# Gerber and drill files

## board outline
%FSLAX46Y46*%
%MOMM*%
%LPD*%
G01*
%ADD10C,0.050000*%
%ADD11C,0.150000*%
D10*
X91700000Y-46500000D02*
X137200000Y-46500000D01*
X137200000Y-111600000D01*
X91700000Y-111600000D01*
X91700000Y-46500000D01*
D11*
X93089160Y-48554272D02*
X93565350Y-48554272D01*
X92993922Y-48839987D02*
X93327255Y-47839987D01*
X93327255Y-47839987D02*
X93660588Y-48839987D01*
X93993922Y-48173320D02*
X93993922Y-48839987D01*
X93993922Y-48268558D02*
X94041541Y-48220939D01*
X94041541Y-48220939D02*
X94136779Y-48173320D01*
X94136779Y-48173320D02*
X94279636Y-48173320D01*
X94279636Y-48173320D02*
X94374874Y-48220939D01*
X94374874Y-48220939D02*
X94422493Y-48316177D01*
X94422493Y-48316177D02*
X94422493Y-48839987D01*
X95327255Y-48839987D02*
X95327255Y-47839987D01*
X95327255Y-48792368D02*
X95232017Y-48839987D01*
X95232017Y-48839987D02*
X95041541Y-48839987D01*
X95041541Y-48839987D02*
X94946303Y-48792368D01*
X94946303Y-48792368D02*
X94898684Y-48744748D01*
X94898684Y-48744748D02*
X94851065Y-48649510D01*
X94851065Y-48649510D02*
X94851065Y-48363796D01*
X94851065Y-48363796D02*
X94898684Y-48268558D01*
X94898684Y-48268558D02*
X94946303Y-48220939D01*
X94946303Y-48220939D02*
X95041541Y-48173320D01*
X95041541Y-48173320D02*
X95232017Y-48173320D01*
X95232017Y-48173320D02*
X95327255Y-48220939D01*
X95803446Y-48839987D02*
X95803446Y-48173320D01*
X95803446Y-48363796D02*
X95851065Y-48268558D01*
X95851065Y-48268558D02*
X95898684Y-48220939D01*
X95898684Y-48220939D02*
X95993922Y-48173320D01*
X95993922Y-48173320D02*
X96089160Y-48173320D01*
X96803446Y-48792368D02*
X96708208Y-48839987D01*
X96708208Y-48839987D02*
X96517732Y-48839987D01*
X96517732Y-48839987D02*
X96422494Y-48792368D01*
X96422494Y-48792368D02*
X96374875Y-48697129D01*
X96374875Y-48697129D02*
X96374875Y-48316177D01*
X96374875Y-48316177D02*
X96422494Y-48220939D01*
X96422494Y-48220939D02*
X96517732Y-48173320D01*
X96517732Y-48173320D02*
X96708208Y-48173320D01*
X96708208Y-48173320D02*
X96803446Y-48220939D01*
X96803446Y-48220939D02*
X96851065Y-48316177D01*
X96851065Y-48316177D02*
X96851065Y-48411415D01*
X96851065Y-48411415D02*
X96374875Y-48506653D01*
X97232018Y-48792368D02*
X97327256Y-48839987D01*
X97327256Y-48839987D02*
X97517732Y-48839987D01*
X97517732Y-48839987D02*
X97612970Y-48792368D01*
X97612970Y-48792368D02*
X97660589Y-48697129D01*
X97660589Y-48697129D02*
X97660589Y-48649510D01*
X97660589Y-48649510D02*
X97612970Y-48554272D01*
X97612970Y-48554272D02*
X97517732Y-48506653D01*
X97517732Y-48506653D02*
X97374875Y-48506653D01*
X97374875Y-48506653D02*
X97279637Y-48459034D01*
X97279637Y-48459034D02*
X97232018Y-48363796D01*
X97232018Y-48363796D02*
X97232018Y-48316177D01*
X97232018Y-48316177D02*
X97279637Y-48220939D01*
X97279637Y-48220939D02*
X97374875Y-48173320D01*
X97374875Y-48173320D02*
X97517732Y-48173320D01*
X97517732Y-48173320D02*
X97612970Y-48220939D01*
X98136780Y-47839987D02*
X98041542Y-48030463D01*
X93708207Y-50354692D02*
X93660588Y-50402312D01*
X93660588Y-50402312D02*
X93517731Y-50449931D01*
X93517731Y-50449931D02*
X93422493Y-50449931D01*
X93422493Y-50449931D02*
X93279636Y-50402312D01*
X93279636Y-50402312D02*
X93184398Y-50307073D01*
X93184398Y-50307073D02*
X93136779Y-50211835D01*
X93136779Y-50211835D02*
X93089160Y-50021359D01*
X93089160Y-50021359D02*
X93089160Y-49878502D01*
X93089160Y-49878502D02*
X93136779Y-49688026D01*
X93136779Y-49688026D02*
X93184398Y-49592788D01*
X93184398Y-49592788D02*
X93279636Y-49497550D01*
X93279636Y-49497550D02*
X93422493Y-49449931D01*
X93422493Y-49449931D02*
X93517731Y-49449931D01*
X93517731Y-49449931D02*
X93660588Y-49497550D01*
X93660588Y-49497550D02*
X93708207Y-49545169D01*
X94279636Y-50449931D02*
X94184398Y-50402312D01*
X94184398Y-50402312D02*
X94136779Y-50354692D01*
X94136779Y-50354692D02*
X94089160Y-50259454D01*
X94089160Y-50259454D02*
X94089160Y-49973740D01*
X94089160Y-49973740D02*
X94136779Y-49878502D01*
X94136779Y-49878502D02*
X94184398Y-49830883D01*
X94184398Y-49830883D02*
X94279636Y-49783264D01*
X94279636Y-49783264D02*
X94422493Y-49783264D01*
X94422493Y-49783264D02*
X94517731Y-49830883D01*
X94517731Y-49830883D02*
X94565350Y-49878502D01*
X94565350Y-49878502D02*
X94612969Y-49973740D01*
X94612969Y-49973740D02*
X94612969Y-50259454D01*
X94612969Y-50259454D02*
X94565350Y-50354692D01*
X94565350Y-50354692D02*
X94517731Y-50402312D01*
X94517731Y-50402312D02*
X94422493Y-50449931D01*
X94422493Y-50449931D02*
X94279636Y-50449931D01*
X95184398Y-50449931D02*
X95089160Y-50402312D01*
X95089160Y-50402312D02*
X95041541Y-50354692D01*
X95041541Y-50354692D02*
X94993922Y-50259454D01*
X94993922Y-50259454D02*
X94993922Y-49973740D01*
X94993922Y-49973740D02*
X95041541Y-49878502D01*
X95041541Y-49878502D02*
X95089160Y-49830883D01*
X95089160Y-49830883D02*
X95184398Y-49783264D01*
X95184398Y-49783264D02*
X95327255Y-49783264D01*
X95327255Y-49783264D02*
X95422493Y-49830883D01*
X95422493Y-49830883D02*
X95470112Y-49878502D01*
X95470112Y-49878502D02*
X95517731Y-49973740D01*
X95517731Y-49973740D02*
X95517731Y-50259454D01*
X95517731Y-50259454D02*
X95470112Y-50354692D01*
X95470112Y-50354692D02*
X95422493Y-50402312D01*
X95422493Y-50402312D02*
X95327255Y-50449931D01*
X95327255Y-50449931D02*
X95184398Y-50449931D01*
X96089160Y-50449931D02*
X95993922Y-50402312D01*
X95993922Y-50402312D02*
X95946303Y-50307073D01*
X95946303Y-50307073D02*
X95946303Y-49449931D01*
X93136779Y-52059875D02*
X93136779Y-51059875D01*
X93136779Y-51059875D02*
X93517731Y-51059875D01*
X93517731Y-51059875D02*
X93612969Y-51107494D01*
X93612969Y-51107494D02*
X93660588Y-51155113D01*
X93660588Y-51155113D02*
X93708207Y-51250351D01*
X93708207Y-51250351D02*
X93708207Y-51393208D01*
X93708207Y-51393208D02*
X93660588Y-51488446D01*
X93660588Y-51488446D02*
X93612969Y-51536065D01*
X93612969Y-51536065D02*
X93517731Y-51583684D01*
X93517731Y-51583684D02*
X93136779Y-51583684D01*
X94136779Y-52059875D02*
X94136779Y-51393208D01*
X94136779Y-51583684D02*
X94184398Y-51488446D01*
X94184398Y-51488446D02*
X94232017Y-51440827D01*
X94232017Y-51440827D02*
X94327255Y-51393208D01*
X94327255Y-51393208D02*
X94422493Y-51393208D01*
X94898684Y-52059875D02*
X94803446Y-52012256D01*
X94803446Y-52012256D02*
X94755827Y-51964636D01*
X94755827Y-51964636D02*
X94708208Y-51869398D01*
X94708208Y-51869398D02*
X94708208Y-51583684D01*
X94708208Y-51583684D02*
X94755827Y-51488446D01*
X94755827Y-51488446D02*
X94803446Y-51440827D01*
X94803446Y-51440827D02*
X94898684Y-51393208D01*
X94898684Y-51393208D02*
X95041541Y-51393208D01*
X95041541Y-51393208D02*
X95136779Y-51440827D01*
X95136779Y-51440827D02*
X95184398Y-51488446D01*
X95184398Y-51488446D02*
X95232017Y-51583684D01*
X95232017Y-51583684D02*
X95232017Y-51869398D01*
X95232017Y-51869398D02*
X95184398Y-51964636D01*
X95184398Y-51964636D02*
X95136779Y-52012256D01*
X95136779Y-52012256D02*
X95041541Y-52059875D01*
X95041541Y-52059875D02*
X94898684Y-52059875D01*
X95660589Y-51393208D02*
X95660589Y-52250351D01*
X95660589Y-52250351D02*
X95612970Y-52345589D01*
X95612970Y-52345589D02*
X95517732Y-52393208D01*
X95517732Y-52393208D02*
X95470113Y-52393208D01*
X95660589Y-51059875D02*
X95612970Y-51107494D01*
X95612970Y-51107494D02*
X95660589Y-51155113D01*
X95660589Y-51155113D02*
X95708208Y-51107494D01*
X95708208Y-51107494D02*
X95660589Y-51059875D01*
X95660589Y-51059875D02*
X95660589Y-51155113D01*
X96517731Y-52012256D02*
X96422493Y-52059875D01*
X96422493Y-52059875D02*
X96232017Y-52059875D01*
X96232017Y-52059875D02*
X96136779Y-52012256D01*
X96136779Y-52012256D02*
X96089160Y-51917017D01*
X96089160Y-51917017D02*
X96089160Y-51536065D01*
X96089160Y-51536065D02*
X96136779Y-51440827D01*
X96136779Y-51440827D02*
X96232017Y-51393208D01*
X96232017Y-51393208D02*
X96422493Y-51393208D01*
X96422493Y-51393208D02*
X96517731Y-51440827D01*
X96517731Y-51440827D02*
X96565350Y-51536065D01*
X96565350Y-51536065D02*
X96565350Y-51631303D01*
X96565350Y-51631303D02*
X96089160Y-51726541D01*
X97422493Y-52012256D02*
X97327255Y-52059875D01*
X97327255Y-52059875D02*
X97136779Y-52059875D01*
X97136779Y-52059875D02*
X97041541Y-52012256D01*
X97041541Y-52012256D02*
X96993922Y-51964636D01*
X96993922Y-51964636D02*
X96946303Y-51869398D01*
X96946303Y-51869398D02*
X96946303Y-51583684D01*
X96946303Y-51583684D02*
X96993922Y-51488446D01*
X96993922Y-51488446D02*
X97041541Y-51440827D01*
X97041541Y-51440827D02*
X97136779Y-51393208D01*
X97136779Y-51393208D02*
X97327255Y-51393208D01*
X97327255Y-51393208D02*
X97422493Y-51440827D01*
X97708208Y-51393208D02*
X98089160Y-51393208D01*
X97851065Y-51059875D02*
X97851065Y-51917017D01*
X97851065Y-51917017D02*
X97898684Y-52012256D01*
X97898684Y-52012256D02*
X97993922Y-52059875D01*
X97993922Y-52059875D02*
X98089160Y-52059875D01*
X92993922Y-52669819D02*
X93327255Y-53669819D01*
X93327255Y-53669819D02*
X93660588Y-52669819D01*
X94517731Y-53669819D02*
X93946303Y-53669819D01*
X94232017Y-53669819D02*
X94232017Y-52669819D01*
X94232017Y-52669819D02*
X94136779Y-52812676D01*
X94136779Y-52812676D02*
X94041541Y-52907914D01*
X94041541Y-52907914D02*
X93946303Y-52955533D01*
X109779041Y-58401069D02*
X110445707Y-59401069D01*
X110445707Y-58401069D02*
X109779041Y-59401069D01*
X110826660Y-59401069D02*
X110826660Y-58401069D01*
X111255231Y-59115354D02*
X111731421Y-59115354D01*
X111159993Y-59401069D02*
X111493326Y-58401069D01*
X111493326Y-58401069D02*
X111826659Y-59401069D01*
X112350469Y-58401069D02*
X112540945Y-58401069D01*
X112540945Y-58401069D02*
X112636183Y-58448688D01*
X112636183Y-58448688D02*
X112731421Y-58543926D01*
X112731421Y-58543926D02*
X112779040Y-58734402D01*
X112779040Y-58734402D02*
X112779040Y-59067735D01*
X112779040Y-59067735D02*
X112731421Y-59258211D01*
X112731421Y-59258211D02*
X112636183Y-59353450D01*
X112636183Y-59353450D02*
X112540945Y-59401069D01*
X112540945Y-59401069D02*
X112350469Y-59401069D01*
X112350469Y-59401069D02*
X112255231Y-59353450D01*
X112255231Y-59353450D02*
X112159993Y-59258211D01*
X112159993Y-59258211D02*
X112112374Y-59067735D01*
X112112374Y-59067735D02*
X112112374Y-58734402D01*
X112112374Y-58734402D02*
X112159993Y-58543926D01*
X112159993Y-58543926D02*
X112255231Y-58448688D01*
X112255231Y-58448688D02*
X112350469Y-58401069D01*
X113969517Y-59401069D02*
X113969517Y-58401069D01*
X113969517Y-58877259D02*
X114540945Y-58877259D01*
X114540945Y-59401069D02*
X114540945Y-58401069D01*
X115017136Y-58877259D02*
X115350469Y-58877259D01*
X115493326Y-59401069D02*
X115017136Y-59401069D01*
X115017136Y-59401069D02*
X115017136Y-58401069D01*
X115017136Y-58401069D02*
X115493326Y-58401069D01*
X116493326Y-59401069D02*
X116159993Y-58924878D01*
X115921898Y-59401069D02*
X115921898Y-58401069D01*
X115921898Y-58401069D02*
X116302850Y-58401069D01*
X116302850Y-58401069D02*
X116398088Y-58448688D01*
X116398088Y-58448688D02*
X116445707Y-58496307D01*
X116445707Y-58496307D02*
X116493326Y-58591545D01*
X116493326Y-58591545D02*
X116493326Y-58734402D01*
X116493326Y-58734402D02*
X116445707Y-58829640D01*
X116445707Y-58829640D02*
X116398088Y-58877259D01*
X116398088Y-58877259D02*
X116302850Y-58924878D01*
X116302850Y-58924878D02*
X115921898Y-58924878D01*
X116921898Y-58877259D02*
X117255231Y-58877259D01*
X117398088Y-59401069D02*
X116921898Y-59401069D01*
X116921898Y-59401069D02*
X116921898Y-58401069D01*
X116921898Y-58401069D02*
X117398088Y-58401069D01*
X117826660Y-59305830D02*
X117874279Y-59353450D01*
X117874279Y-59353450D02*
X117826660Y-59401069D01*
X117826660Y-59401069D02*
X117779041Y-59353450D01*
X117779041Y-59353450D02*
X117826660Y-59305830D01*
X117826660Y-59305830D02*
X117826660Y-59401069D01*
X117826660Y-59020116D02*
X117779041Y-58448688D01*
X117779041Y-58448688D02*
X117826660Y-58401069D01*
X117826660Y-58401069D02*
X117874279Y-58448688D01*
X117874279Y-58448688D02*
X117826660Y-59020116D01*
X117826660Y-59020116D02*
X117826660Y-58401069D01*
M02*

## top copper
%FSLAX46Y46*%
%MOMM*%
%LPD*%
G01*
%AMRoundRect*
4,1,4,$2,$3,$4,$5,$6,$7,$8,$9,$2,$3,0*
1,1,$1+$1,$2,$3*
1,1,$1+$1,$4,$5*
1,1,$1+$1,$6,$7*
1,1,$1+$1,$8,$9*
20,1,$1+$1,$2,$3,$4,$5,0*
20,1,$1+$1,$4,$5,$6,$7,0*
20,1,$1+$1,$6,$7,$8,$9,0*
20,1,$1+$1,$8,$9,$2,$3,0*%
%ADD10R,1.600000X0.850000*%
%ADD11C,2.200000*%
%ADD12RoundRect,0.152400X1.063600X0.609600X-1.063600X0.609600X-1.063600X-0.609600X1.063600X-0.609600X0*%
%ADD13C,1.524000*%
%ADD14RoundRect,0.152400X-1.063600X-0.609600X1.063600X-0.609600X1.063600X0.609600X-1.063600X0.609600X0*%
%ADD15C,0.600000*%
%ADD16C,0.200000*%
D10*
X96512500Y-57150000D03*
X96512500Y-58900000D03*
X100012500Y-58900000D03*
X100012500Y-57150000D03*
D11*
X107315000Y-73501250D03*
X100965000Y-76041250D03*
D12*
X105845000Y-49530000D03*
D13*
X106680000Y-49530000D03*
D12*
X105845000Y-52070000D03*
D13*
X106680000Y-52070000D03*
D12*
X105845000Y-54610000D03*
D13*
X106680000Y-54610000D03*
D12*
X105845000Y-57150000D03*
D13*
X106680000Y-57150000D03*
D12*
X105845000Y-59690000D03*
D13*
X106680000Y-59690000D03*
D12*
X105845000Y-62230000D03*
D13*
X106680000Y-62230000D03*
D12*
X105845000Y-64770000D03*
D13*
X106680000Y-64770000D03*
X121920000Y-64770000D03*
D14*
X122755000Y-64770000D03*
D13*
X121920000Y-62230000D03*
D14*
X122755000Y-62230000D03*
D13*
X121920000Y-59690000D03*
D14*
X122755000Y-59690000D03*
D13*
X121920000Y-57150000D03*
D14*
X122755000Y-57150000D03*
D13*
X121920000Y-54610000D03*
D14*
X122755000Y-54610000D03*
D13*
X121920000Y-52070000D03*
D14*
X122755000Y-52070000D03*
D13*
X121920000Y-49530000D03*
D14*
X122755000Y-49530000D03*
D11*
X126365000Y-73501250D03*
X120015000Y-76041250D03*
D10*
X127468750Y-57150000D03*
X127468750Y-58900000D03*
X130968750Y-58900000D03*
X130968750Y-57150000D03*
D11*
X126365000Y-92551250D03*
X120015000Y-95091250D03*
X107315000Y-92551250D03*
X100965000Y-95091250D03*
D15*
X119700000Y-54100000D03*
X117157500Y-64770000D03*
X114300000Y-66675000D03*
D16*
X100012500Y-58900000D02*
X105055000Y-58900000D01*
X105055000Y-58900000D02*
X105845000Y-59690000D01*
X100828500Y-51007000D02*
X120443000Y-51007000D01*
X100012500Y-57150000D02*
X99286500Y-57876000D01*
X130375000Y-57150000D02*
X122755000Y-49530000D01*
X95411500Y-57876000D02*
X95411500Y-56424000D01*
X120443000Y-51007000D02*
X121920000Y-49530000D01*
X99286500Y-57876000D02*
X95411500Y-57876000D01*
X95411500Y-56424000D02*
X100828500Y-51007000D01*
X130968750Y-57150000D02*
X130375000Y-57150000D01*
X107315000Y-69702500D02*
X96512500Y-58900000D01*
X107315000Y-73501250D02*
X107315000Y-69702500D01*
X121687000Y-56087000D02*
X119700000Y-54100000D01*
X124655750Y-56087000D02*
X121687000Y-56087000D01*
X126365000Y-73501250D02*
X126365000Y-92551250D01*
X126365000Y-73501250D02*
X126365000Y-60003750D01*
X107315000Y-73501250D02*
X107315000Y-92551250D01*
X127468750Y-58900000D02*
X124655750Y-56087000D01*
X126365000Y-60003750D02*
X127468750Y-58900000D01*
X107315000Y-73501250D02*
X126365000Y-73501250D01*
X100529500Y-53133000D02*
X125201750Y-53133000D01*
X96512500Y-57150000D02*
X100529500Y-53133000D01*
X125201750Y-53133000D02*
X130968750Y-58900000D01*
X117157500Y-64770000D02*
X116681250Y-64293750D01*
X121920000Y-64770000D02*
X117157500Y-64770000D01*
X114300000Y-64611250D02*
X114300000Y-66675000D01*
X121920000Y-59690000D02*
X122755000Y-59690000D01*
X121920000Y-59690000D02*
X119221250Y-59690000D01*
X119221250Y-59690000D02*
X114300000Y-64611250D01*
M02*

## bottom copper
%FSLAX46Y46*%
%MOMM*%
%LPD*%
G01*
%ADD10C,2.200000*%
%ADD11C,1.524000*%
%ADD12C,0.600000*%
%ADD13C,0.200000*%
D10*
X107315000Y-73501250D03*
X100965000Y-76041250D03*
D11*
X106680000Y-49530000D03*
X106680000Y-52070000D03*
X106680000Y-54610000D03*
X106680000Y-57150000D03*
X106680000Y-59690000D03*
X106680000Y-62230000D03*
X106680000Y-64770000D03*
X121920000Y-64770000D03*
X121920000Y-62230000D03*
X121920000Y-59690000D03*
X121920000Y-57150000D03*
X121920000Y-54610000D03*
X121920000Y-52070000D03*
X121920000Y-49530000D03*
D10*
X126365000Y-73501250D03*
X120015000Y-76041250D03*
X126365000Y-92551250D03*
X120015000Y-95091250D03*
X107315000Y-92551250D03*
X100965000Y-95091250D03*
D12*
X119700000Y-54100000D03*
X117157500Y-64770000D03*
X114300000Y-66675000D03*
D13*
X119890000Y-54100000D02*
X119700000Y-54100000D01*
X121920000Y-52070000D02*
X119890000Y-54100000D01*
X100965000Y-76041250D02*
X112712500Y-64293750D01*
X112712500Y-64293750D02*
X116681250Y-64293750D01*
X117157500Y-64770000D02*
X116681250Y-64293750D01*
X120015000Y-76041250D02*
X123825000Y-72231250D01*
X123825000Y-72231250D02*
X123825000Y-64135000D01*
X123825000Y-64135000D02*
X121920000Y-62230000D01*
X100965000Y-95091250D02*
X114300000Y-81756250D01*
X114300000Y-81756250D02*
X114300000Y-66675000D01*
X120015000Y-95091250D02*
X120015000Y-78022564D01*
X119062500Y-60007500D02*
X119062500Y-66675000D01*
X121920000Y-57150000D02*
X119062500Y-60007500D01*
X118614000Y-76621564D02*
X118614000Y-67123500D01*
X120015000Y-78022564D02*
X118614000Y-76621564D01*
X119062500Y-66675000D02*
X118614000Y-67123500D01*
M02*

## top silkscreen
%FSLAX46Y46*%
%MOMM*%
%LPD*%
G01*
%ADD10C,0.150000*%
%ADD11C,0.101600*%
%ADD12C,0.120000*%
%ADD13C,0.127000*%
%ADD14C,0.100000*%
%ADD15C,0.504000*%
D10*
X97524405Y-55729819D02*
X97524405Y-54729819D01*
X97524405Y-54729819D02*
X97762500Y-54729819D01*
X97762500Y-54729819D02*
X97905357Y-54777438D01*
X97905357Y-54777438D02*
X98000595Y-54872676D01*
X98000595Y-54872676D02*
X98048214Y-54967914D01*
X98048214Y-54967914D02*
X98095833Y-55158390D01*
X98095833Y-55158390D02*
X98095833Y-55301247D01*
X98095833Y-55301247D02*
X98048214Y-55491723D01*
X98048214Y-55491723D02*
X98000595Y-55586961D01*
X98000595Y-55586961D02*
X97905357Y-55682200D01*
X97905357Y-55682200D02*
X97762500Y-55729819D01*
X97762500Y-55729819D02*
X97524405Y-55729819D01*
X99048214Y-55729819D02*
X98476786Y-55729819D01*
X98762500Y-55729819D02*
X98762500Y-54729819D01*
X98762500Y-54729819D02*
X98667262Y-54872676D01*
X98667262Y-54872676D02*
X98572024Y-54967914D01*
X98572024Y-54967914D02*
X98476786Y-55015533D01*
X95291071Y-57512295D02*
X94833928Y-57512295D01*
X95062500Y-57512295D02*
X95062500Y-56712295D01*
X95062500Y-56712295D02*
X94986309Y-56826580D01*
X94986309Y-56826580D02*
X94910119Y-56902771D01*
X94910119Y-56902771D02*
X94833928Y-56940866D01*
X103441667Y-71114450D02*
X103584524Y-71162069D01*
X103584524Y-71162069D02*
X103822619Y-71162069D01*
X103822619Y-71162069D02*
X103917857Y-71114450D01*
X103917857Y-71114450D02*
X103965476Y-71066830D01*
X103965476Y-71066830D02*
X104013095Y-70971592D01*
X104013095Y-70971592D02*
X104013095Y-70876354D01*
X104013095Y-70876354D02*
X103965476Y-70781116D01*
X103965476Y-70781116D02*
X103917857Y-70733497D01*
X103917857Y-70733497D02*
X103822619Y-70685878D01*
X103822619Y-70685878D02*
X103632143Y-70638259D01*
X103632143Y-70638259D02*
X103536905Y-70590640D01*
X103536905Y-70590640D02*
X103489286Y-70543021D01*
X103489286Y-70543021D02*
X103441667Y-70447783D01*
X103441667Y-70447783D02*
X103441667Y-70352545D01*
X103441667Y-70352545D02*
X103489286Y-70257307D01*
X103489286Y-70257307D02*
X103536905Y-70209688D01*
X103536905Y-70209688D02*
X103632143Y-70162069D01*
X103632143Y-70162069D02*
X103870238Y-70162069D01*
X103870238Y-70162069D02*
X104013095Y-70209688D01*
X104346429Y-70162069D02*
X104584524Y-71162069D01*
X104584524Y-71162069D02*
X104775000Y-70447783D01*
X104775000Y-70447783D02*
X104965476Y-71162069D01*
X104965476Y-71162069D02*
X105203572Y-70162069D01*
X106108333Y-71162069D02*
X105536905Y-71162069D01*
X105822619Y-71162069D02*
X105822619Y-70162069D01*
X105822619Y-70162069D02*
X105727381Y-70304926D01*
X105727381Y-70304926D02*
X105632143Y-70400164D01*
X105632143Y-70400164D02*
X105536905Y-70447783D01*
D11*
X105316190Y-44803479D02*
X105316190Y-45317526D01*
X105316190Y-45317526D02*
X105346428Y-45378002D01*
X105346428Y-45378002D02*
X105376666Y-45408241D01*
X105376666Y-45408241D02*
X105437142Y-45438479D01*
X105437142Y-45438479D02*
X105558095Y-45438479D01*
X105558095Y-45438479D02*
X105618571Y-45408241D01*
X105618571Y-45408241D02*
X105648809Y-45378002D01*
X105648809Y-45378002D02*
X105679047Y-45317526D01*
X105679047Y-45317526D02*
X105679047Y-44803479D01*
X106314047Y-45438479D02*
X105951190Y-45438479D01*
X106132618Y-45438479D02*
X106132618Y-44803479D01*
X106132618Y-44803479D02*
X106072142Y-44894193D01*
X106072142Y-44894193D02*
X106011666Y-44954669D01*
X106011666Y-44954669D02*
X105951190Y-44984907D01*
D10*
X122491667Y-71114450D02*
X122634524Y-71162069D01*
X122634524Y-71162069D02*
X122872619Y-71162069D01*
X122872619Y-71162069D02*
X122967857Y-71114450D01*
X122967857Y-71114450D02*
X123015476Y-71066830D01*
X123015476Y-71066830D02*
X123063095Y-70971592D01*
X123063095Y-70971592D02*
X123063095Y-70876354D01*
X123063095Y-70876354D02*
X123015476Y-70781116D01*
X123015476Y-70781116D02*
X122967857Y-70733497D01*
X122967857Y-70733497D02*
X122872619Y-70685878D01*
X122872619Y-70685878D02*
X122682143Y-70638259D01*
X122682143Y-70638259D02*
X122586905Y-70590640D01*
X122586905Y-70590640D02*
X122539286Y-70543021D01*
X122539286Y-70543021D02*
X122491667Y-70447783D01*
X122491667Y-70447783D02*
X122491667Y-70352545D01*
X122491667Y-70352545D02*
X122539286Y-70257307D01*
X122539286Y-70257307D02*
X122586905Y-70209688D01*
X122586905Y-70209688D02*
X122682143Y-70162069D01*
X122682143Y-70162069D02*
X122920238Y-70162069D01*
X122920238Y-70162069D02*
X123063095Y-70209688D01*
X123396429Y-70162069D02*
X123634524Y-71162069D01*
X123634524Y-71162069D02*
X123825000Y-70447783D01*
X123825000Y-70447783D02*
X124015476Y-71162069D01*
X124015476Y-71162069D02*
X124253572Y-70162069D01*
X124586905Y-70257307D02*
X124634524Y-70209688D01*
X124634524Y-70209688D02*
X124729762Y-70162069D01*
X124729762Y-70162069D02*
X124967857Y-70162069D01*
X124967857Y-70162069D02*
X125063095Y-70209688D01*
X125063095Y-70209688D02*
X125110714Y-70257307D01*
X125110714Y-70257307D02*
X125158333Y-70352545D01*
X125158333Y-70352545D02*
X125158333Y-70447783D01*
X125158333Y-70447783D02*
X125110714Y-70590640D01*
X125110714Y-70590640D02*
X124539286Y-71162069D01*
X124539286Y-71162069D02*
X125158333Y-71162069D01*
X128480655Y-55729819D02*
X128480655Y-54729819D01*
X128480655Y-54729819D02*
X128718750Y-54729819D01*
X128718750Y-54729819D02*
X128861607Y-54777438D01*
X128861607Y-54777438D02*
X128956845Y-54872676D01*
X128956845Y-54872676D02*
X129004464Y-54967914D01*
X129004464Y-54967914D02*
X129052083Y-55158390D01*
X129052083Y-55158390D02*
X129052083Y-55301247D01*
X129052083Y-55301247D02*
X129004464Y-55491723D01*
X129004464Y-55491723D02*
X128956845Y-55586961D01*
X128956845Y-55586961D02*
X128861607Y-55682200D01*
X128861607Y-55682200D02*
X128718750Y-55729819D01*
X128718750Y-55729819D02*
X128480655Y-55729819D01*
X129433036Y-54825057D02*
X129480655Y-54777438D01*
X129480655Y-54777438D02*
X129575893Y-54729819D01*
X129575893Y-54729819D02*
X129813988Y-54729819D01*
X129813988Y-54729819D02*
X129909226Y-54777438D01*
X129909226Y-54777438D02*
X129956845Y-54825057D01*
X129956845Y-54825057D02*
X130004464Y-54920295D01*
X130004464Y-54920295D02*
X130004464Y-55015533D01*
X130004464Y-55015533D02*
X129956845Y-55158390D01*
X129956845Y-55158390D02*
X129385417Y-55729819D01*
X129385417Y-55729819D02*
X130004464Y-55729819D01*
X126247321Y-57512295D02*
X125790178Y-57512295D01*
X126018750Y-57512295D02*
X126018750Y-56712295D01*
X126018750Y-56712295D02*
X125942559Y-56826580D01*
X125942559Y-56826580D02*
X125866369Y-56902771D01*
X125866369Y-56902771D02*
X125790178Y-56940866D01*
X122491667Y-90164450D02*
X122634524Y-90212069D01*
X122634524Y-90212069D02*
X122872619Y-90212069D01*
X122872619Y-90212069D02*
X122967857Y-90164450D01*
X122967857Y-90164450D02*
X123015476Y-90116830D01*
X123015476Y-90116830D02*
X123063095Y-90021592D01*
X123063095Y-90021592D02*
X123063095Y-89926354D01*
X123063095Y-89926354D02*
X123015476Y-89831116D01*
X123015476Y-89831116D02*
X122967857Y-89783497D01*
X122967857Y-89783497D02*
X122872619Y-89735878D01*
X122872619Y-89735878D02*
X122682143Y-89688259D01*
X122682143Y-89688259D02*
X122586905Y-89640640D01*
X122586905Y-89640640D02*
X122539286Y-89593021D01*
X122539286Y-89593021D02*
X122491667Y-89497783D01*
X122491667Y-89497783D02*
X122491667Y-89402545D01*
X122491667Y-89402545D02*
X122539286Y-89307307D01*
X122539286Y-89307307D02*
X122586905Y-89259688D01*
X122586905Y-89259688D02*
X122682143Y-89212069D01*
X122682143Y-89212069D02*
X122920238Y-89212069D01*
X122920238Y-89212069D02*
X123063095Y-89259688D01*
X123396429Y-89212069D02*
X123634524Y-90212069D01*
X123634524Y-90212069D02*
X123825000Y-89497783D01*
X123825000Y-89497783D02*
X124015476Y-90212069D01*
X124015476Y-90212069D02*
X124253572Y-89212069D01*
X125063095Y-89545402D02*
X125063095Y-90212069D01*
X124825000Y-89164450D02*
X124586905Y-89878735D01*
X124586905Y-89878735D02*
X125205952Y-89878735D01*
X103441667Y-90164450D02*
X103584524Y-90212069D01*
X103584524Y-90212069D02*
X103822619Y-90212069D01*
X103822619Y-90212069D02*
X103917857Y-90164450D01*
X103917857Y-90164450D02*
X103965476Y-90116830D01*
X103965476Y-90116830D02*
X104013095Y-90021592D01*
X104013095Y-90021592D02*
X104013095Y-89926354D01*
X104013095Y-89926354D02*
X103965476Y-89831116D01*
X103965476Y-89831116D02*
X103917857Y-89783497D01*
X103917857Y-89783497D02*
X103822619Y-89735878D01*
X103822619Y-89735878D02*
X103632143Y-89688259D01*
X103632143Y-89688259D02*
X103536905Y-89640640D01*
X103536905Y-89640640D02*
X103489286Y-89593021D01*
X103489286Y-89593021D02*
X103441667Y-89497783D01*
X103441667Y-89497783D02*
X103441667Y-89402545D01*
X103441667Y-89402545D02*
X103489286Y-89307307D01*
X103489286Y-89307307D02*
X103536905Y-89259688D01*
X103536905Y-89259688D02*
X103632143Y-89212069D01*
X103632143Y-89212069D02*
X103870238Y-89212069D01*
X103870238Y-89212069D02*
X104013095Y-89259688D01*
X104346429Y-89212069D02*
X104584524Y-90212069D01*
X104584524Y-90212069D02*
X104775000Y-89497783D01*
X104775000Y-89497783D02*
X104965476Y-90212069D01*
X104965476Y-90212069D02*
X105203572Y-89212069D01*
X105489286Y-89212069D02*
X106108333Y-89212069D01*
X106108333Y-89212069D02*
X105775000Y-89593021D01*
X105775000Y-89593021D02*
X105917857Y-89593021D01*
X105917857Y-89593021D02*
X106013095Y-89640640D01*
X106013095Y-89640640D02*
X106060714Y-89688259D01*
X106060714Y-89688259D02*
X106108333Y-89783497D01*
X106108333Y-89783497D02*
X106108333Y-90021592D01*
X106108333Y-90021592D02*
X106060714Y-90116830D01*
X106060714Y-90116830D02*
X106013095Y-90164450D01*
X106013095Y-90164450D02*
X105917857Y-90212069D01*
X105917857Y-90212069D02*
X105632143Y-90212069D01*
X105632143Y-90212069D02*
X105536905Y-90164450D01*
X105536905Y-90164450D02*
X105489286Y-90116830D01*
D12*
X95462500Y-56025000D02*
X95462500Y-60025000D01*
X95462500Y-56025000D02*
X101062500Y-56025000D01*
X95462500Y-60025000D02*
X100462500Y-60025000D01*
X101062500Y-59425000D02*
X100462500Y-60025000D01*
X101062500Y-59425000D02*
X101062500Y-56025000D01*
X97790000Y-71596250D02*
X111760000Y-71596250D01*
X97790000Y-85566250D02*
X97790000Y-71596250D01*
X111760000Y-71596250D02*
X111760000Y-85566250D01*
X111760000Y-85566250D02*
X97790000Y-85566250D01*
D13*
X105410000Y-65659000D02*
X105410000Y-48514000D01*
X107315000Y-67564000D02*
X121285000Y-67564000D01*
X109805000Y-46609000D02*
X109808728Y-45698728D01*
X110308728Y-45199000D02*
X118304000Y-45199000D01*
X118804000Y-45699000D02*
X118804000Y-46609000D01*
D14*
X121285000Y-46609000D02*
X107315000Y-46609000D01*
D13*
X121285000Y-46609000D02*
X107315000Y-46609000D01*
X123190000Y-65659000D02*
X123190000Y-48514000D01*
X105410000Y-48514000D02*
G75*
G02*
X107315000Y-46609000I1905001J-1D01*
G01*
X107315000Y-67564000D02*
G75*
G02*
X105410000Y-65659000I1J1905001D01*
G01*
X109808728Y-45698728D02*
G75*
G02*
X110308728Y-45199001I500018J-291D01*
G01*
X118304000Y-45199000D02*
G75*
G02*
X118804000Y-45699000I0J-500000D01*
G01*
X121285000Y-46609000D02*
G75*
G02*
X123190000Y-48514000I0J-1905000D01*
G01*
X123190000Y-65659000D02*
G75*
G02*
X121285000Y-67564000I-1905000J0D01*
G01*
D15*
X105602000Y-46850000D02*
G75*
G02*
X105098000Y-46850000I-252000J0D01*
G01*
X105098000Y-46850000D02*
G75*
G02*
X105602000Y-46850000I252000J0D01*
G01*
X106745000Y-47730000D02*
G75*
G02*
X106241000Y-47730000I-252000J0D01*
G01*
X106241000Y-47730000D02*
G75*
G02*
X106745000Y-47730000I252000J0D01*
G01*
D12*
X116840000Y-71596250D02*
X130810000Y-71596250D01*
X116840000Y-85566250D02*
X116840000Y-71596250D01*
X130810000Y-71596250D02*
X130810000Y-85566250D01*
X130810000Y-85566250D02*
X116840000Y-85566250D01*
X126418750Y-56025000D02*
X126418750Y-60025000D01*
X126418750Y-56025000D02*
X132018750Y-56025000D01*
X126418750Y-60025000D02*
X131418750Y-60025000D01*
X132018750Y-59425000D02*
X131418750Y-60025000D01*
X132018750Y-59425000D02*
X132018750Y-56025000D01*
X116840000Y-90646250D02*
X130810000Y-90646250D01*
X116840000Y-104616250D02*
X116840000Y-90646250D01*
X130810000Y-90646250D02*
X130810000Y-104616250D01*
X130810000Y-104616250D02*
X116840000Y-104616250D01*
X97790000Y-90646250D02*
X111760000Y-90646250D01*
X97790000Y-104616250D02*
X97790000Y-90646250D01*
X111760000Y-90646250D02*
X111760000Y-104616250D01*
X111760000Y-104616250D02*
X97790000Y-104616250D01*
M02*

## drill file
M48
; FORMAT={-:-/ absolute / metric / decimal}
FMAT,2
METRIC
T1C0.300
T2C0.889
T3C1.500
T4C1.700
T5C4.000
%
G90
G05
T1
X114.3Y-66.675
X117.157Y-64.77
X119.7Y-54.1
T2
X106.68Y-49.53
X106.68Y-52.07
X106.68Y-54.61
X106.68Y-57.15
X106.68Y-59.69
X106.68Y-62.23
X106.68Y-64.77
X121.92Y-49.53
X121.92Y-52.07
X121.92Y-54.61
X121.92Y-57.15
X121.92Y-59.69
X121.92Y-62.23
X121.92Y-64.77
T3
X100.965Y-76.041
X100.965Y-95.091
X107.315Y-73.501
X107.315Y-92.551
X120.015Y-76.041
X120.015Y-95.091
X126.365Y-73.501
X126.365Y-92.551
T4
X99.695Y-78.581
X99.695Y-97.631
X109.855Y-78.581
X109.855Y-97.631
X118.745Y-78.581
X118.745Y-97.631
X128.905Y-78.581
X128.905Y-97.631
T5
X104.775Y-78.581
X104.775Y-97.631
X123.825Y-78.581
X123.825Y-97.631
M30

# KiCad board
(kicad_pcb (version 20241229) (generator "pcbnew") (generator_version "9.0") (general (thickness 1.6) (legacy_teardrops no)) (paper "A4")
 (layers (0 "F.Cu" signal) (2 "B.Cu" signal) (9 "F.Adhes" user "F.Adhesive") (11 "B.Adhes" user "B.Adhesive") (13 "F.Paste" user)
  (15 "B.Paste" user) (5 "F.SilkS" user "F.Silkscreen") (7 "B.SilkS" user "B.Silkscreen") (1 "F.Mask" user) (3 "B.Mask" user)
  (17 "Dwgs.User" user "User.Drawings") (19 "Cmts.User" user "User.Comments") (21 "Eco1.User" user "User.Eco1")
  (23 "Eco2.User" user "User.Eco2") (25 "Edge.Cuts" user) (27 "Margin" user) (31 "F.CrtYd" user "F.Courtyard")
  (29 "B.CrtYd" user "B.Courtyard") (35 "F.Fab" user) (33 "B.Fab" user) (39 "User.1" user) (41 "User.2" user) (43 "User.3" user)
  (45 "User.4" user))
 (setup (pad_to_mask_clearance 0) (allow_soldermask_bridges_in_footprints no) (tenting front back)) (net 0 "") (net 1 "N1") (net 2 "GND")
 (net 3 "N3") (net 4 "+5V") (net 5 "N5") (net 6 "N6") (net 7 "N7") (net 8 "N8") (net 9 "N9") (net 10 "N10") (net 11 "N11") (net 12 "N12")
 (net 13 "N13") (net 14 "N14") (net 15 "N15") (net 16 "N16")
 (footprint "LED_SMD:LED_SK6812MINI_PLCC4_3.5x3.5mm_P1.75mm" (layer "F.Cu") (at 98.2625 58.025)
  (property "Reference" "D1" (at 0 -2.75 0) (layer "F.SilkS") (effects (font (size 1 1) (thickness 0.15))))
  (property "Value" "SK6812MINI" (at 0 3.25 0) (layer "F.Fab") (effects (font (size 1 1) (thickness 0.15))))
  (fp_line (start -2.8 -2) (end -2.8 2) (stroke (width 0.12) (type default)) (layer "F.SilkS"))
  (fp_line (start -2.8 -2) (end 2.8 -2) (stroke (width 0.12) (type solid)) (layer "F.SilkS"))
  (fp_line (start -2.8 2) (end 2.2 2) (stroke (width 0.12) (type solid)) (layer "F.SilkS"))
  (fp_line (start 2.8 1.4) (end 2.2 2) (stroke (width 0.12) (type default)) (layer "F.SilkS"))
  (fp_line (start 2.8 1.4) (end 2.8 -2) (stroke (width 0.12) (type solid)) (layer "F.SilkS"))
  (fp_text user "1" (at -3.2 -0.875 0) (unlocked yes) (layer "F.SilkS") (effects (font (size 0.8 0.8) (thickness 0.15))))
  (pad "1" smd rect (at -1.75 -0.875) (size 1.6 0.85) (layers "F.Cu" "F.Mask" "F.Paste") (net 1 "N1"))
  (pad "2" smd rect (at -1.75 0.875) (size 1.6 0.85) (layers "F.Cu" "F.Mask" "F.Paste") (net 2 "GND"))
  (pad "3" smd rect (at 1.75 0.875) (size 1.6 0.85) (layers "F.Cu" "F.Mask" "F.Paste") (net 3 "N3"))
  (pad "4" smd rect (at 1.75 -0.875) (size 1.6 0.85) (layers "F.Cu" "F.Mask" "F.Paste") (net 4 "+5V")))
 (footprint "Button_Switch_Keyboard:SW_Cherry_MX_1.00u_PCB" (layer "F.Cu") (at 107.315 73.50125)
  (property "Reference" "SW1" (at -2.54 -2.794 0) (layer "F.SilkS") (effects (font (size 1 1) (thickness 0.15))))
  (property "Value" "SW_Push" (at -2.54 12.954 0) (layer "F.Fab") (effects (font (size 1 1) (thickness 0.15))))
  (fp_line (start -9.525 -1.905) (end 4.445 -1.905) (stroke (width 0.12) (type solid)) (layer "F.SilkS"))
  (fp_line (start -9.525 12.065) (end -9.525 -1.905) (stroke (width 0.12) (type solid)) (layer "F.SilkS"))
  (fp_line (start 4.445 -1.905) (end 4.445 12.065) (stroke (width 0.12) (type solid)) (layer "F.SilkS"))
  (fp_line (start 4.445 12.065) (end -9.525 12.065) (stroke (width 0.12) (type solid)) (layer "F.SilkS"))
  (pad "" np_thru_hole circle (at -7.62 5.08) (size 1.7 1.7) (drill 1.7) (layers "*.Cu" "*.Mask"))
  (pad "" np_thru_hole circle (at -2.54 5.08) (size 4 4) (drill 4) (layers "*.Cu" "*.Mask"))
  (pad "" np_thru_hole circle (at 2.54 5.08) (size 1.7 1.7) (drill 1.7) (layers "*.Cu" "*.Mask"))
  (pad "1" thru_hole circle (at 0 0) (size 2.2 2.2) (drill 1.5) (layers "*.Cu" "*.Mask") (remove_unused_layers no) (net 2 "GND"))
  (pad "2" thru_hole circle (at -6.35 2.54) (size 2.2 2.2) (drill 1.5) (layers "*.Cu" "*.Mask") (remove_unused_layers no) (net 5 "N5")))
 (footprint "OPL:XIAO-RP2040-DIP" (layer "F.Cu") (at 114.3 57.15)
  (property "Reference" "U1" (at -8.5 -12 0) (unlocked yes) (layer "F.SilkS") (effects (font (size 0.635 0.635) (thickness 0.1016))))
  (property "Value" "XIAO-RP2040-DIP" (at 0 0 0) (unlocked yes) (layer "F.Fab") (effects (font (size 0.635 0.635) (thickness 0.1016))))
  (fp_line (start -8.89 8.509) (end -8.89 -8.636) (stroke (width 0.127) (type solid)) (layer "F.SilkS"))
  (fp_line (start -6.985 10.414) (end 6.985 10.414) (stroke (width 0.127) (type solid)) (layer "F.SilkS"))
  (fp_line (start -4.495 -10.541) (end -4.491272 -11.451272) (stroke (width 0.127) (type solid)) (layer "F.SilkS"))
  (fp_line (start -3.991272 -11.951) (end 4.004 -11.951) (stroke (width 0.127) (type solid)) (layer "F.SilkS"))
  (fp_line (start 4.504 -11.451) (end 4.504 -10.541) (stroke (width 0.127) (type solid)) (layer "F.SilkS"))
  (fp_line (start 6.985 -10.541) (end -6.985 -10.541) (stroke (width 0.1) (type solid)) (layer "F.SilkS"))
  (fp_line (start 6.985 -10.541) (end -6.985 -10.541) (stroke (width 0.127) (type solid)) (layer "F.SilkS"))
  (fp_line (start 8.89 8.509) (end 8.89 -8.636) (stroke (width 0.127) (type solid)) (layer "F.SilkS"))
  (fp_arc (start -8.89 -8.636) (mid -8.332038 -9.983038) (end -6.985 -10.541) (stroke (width 0.127) (type solid)) (layer "F.SilkS"))
  (fp_arc (start -6.985 10.414) (mid -8.332038 9.856038) (end -8.89 8.509) (stroke (width 0.127) (type solid)) (layer "F.SilkS"))
  (fp_arc (start -4.491272 -11.451272) (mid -4.344728 -11.80464) (end -3.991272 -11.951) (stroke (width 0.127) (type default))
   (layer "F.SilkS"))
  (fp_arc (start 4.004 -11.951) (mid 4.357553 -11.804553) (end 4.504 -11.451) (stroke (width 0.127) (type default)) (layer "F.SilkS"))
  (fp_arc (start 6.985 -10.541) (mid 8.332038 -9.983038) (end 8.89 -8.636) (stroke (width 0.127) (type solid)) (layer "F.SilkS"))
  (fp_arc (start 8.89 8.509) (mid 8.332038 9.856038) (end 6.985 10.414) (stroke (width 0.127) (type solid)) (layer "F.SilkS"))
  (fp_circle (center -8.95 -10.3) (end -8.95 -10.554) (stroke (width 0.5) (type solid)) (fill yes) (layer "F.SilkS"))
  (fp_circle (center -7.807 -9.42) (end -7.807 -9.674) (stroke (width 0.5) (type solid)) (fill yes) (layer "F.SilkS"))
  (pad "1" smd roundrect (at -8.455 -7.62 180) (size 2.432 1.524) (layers "F.Cu" "F.Mask") (roundrect_rratio 0.1) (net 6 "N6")
   (thermal_bridge_angle 45))
  (pad "1" thru_hole circle (at -7.62 -7.62 180) (size 1.524 1.524) (drill 0.889) (layers "*.Cu" "*.Mask") (remove_unused_layers no)
   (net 6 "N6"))
  (pad "2" smd roundrect (at -8.455 -5.08 180) (size 2.432 1.524) (layers "F.Cu" "F.Mask") (roundrect_rratio 0.1) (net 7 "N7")
   (thermal_bridge_angle 45))
  (pad "2" thru_hole circle (at -7.62 -5.08 180) (size 1.524 1.524) (drill 0.889) (layers "*.Cu" "*.Mask") (remove_unused_layers no)
   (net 7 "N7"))
  (pad "3" smd roundrect (at -8.455 -2.54 180) (size 2.432 1.524) (layers "F.Cu" "F.Mask") (roundrect_rratio 0.1) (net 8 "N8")
   (thermal_bridge_angle 45))
  (pad "3" thru_hole circle (at -7.62 -2.54 180) (size 1.524 1.524) (drill 0.889) (layers "*.Cu" "*.Mask") (remove_unused_layers no)
   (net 8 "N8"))
  (pad "4" smd roundrect (at -8.455 0 180) (size 2.432 1.524) (layers "F.Cu" "F.Mask") (roundrect_rratio 0.1) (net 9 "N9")
   (thermal_bridge_angle 45))
  (pad "4" thru_hole circle (at -7.62 0 180) (size 1.524 1.524) (drill 0.889) (layers "*.Cu" "*.Mask") (remove_unused_layers no)
   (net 9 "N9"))
  (pad "5" smd roundrect (at -8.455 2.54 180) (size 2.432 1.524) (layers "F.Cu" "F.Mask") (roundrect_rratio 0.1) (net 3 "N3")
   (thermal_bridge_angle 45))
  (pad "5" thru_hole circle (at -7.62 2.54 180) (size 1.524 1.524) (drill 0.889) (layers "*.Cu" "*.Mask") (remove_unused_layers no)
   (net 3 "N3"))
  (pad "6" smd roundrect (at -8.455 5.08 180) (size 2.432 1.524) (layers "F.Cu" "F.Mask") (roundrect_rratio 0.1) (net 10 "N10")
   (thermal_bridge_angle 45))
  (pad "6" thru_hole circle (at -7.62 5.08 180) (size 1.524 1.524) (drill 0.889) (layers "*.Cu" "*.Mask") (remove_unused_layers no)
   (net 10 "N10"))
  (pad "7" smd roundrect (at -8.455 7.62 180) (size 2.432 1.524) (layers "F.Cu" "F.Mask") (roundrect_rratio 0.1) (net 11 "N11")
   (thermal_bridge_angle 45))
  (pad "7" thru_hole circle (at -7.62 7.62 180) (size 1.524 1.524) (drill 0.889) (layers "*.Cu" "*.Mask") (remove_unused_layers no)
   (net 11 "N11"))
  (pad "8" thru_hole circle (at 7.62 7.62) (size 1.524 1.524) (drill 0.889) (layers "*.Cu" "*.Mask") (remove_unused_layers no) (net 5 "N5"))
  (pad "8" smd roundrect (at 8.455 7.62) (size 2.432 1.524) (layers "F.Cu" "F.Mask") (roundrect_rratio 0.1) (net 5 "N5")
   (thermal_bridge_angle 45))
  (pad "9" thru_hole circle (at 7.62 5.08) (size 1.524 1.524) (drill 0.889) (layers "*.Cu" "*.Mask") (remove_unused_layers no)
   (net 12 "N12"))
  (pad "9" smd roundrect (at 8.455 5.08) (size 2.432 1.524) (layers "F.Cu" "F.Mask") (roundrect_rratio 0.1) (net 12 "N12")
   (thermal_bridge_angle 45))
  (pad "10" thru_hole circle (at 7.62 2.54) (size 1.524 1.524) (drill 0.889) (layers "*.Cu" "*.Mask") (remove_unused_layers no)
   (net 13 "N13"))
  (pad "10" smd roundrect (at 8.455 2.54) (size 2.432 1.524) (layers "F.Cu" "F.Mask") (roundrect_rratio 0.1) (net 13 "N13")
   (thermal_bridge_angle 45))
  (pad "11" thru_hole circle (at 7.62 0) (size 1.524 1.524) (drill 0.889) (layers "*.Cu" "*.Mask") (remove_unused_layers no) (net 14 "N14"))
  (pad "11" smd roundrect (at 8.455 0) (size 2.432 1.524) (layers "F.Cu" "F.Mask") (roundrect_rratio 0.1) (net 14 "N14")
   (thermal_bridge_angle 45))
  (pad "12" thru_hole circle (at 7.62 -2.54) (size 1.524 1.524) (drill 0.889) (layers "*.Cu" "*.Mask") (remove_unused_layers no)
   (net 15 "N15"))
  (pad "12" smd roundrect (at 8.455 -2.54) (size 2.432 1.524) (layers "F.Cu" "F.Mask") (roundrect_rratio 0.1) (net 15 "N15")
   (thermal_bridge_angle 45))
  (pad "13" thru_hole circle (at 7.62 -5.08) (size 1.524 1.524) (drill 0.889) (layers "*.Cu" "*.Mask") (remove_unused_layers no)
   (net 2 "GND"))
  (pad "13" smd roundrect (at 8.455 -5.08) (size 2.432 1.524) (layers "F.Cu" "F.Mask") (roundrect_rratio 0.1) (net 2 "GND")
   (thermal_bridge_angle 45))
  (pad "14" thru_hole circle (at 7.62 -7.62) (size 1.524 1.524) (drill 0.889) (layers "*.Cu" "*.Mask") (remove_unused_layers no)
   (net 4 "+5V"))
  (pad "14" smd roundrect (at 8.455 -7.62) (size 2.432 1.524) (layers "F.Cu" "F.Mask") (roundrect_rratio 0.1) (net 4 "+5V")
   (thermal_bridge_angle 45)))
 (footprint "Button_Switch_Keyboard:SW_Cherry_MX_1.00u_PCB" (layer "F.Cu") (at 126.365 73.50125)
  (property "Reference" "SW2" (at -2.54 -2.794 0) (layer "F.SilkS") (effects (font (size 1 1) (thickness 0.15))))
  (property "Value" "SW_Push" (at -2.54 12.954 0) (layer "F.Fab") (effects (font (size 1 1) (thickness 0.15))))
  (fp_line (start -9.525 -1.905) (end 4.445 -1.905) (stroke (width 0.12) (type solid)) (layer "F.SilkS"))
  (fp_line (start -9.525 12.065) (end -9.525 -1.905) (stroke (width 0.12) (type solid)) (layer "F.SilkS"))
  (fp_line (start 4.445 -1.905) (end 4.445 12.065) (stroke (width 0.12) (type solid)) (layer "F.SilkS"))
  (fp_line (start 4.445 12.065) (end -9.525 12.065) (stroke (width 0.12) (type solid)) (layer "F.SilkS"))
  (pad "" np_thru_hole circle (at -7.62 5.08) (size 1.7 1.7) (drill 1.7) (layers "*.Cu" "*.Mask"))
  (pad "" np_thru_hole circle (at -2.54 5.08) (size 4 4) (drill 4) (layers "*.Cu" "*.Mask"))
  (pad "" np_thru_hole circle (at 2.54 5.08) (size 1.7 1.7) (drill 1.7) (layers "*.Cu" "*.Mask"))
  (pad "1" thru_hole circle (at 0 0) (size 2.2 2.2) (drill 1.5) (layers "*.Cu" "*.Mask") (remove_unused_layers no) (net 2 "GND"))
  (pad "2" thru_hole circle (at -6.35 2.54) (size 2.2 2.2) (drill 1.5) (layers "*.Cu" "*.Mask") (remove_unused_layers no) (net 12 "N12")))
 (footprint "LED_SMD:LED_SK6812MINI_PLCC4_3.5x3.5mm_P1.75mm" (layer "F.Cu") (at 129.21875 58.025)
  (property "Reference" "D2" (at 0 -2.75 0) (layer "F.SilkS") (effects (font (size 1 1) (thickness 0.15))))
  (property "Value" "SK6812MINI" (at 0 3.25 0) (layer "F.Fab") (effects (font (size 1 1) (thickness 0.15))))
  (fp_line (start -2.8 -2) (end -2.8 2) (stroke (width 0.12) (type default)) (layer "F.SilkS"))
  (fp_line (start -2.8 -2) (end 2.8 -2) (stroke (width 0.12) (type solid)) (layer "F.SilkS"))
  (fp_line (start -2.8 2) (end 2.2 2) (stroke (width 0.12) (type solid)) (layer "F.SilkS"))
  (fp_line (start 2.8 1.4) (end 2.2 2) (stroke (width 0.12) (type default)) (layer "F.SilkS"))
  (fp_line (start 2.8 1.4) (end 2.8 -2) (stroke (width 0.12) (type solid)) (layer "F.SilkS"))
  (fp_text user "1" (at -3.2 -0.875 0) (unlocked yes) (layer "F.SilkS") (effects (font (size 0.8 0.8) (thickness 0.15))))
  (pad "1" smd rect (at -1.75 -0.875) (size 1.6 0.85) (layers "F.Cu" "F.Mask" "F.Paste") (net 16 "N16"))
  (pad "2" smd rect (at -1.75 0.875) (size 1.6 0.85) (layers "F.Cu" "F.Mask" "F.Paste") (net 2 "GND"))
  (pad "3" smd rect (at 1.75 0.875) (size 1.6 0.85) (layers "F.Cu" "F.Mask" "F.Paste") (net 1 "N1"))
  (pad "4" smd rect (at 1.75 -0.875) (size 1.6 0.85) (layers "F.Cu" "F.Mask" "F.Paste") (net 4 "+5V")))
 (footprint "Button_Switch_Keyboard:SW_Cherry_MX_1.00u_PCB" (layer "F.Cu") (at 126.365 92.55125)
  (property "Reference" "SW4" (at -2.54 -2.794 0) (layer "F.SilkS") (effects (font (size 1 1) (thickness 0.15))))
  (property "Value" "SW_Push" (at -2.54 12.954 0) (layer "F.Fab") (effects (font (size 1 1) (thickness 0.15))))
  (fp_line (start -9.525 -1.905) (end 4.445 -1.905) (stroke (width 0.12) (type solid)) (layer "F.SilkS"))
  (fp_line (start -9.525 12.065) (end -9.525 -1.905) (stroke (width 0.12) (type solid)) (layer "F.SilkS"))
  (fp_line (start 4.445 -1.905) (end 4.445 12.065) (stroke (width 0.12) (type solid)) (layer "F.SilkS"))
  (fp_line (start 4.445 12.065) (end -9.525 12.065) (stroke (width 0.12) (type solid)) (layer "F.SilkS"))
  (pad "" np_thru_hole circle (at -7.62 5.08) (size 1.7 1.7) (drill 1.7) (layers "*.Cu" "*.Mask"))
  (pad "" np_thru_hole circle (at -2.54 5.08) (size 4 4) (drill 4) (layers "*.Cu" "*.Mask"))
  (pad "" np_thru_hole circle (at 2.54 5.08) (size 1.7 1.7) (drill 1.7) (layers "*.Cu" "*.Mask"))
  (pad "1" thru_hole circle (at 0 0) (size 2.2 2.2) (drill 1.5) (layers "*.Cu" "*.Mask") (remove_unused_layers no) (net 2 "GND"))
  (pad "2" thru_hole circle (at -6.35 2.54) (size 2.2 2.2) (drill 1.5) (layers "*.Cu" "*.Mask") (remove_unused_layers no) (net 14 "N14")))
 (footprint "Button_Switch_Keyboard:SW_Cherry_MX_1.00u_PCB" (layer "F.Cu") (at 107.315 92.55125)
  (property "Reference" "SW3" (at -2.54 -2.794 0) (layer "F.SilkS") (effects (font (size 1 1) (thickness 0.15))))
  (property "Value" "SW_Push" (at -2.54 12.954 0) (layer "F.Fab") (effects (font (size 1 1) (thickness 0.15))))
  (fp_line (start -9.525 -1.905) (end 4.445 -1.905) (stroke (width 0.12) (type solid)) (layer "F.SilkS"))
  (fp_line (start -9.525 12.065) (end -9.525 -1.905) (stroke (width 0.12) (type solid)) (layer "F.SilkS"))
  (fp_line (start 4.445 -1.905) (end 4.445 12.065) (stroke (width 0.12) (type solid)) (layer "F.SilkS"))
  (fp_line (start 4.445 12.065) (end -9.525 12.065) (stroke (width 0.12) (type solid)) (layer "F.SilkS"))
  (pad "" np_thru_hole circle (at -7.62 5.08) (size 1.7 1.7) (drill 1.7) (layers "*.Cu" "*.Mask"))
  (pad "" np_thru_hole circle (at -2.54 5.08) (size 4 4) (drill 4) (layers "*.Cu" "*.Mask"))
  (pad "" np_thru_hole circle (at 2.54 5.08) (size 1.7 1.7) (drill 1.7) (layers "*.Cu" "*.Mask"))
  (pad "1" thru_hole circle (at 0 0) (size 2.2 2.2) (drill 1.5) (layers "*.Cu" "*.Mask") (remove_unused_layers no) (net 2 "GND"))
  (pad "2" thru_hole circle (at -6.35 2.54) (size 2.2 2.2) (drill 1.5) (layers "*.Cu" "*.Mask") (remove_unused_layers no) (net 13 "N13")))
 (gr_rect (start 91.7 46.5) (end 137.2 111.6) (stroke (width 0.05) (type default)) (fill no) (layer "Edge.Cuts"))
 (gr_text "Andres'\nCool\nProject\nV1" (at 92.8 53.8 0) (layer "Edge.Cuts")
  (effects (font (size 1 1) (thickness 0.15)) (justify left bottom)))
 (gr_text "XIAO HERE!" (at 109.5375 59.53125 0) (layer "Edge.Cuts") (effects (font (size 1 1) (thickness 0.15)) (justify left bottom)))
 (segment (start 100.0125 58.9) (end 105.055 58.9) (width 0.2) (layer "F.Cu") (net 3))
 (segment (start 105.055 58.9) (end 105.845 59.69) (width 0.2) (layer "F.Cu") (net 3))
 (segment (start 100.8285 51.007) (end 120.443 51.007) (width 0.2) (layer "F.Cu") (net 4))
 (segment (start 100.0125 57.15) (end 99.2865 57.876) (width 0.2) (layer "F.Cu") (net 4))
 (segment (start 130.375 57.15) (end 122.755 49.53) (width 0.2) (layer "F.Cu") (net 4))
 (segment (start 95.4115 57.876) (end 95.4115 56.424) (width 0.2) (layer "F.Cu") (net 4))
 (segment (start 120.443 51.007) (end 121.92 49.53) (width 0.2) (layer "F.Cu") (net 4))
 (segment (start 99.2865 57.876) (end 95.4115 57.876) (width 0.2) (layer "F.Cu") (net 4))
 (segment (start 95.4115 56.424) (end 100.8285 51.007) (width 0.2) (layer "F.Cu") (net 4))
 (segment (start 130.96875 57.15) (end 130.375 57.15) (width 0.2) (layer "F.Cu") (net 4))
 (segment (start 107.315 69.7025) (end 96.5125 58.9) (width 0.2) (layer "F.Cu") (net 2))
 (segment (start 107.315 73.50125) (end 107.315 69.7025) (width 0.2) (layer "F.Cu") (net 2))
 (segment (start 121.687 56.087) (end 119.7 54.1) (width 0.2) (layer "F.Cu") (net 2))
 (segment (start 124.65575 56.087) (end 121.687 56.087) (width 0.2) (layer "F.Cu") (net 2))
 (segment (start 126.365 73.50125) (end 126.365 92.55125) (width 0.2) (layer "F.Cu") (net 2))
 (segment (start 126.365 73.50125) (end 126.365 60.00375) (width 0.2) (layer "F.Cu") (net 2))
 (segment (start 107.315 73.50125) (end 107.315 92.55125) (width 0.2) (layer "F.Cu") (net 2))
 (segment (start 127.46875 58.9) (end 124.65575 56.087) (width 0.2) (layer "F.Cu") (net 2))
 (segment (start 126.365 60.00375) (end 127.46875 58.9) (width 0.2) (layer "F.Cu") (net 2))
 (segment (start 107.315 73.50125) (end 126.365 73.50125) (width 0.2) (layer "F.Cu") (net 2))
 (via (at 119.7 54.1) (size 0.6) (drill 0.3) (layers "F.Cu" "B.Cu") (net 2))
 (segment (start 119.89 54.1) (end 119.7 54.1) (width 0.2) (layer "B.Cu") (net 2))
 (segment (start 121.92 52.07) (end 119.89 54.1) (width 0.2) (layer "B.Cu") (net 2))
 (segment (start 100.5295 53.133) (end 125.20175 53.133) (width 0.2) (layer "F.Cu") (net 1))
 (segment (start 96.5125 57.15) (end 100.5295 53.133) (width 0.2) (layer "F.Cu") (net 1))
 (segment (start 125.20175 53.133) (end 130.96875 58.9) (width 0.2) (layer "F.Cu") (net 1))
 (segment (start 117.1575 64.77) (end 116.68125 64.29375) (width 0.2) (layer "F.Cu") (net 5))
 (segment (start 121.92 64.77) (end 117.1575 64.77) (width 0.2) (layer "F.Cu") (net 5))
 (via (at 117.1575 64.77) (size 0.6) (drill 0.3) (layers "F.Cu" "B.Cu") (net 5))
 (segment (start 100.965 76.04125) (end 112.7125 64.29375) (width 0.2) (layer "B.Cu") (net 5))
 (segment (start 112.7125 64.29375) (end 116.68125 64.29375) (width 0.2) (layer "B.Cu") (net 5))
 (segment (start 117.1575 64.77) (end 116.68125 64.29375) (width 0.2) (layer "B.Cu") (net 5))
 (segment (start 120.015 76.04125) (end 123.825 72.23125) (width 0.2) (layer "B.Cu") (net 12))
 (segment (start 123.825 72.23125) (end 123.825 64.135) (width 0.2) (layer "B.Cu") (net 12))
 (segment (start 123.825 64.135) (end 121.92 62.23) (width 0.2) (layer "B.Cu") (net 12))
 (segment (start 114.3 64.61125) (end 114.3 66.675) (width 0.2) (layer "F.Cu") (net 13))
 (segment (start 121.92 59.69) (end 122.755 59.69) (width 0.2) (layer "F.Cu") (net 13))
 (segment (start 121.92 59.69) (end 119.22125 59.69) (width 0.2) (layer "F.Cu") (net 13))
 (segment (start 119.22125 59.69) (end 114.3 64.61125) (width 0.2) (layer "F.Cu") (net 13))
 (via (at 114.3 66.675) (size 0.6) (drill 0.3) (layers "F.Cu" "B.Cu") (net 13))
 (segment (start 100.965 95.09125) (end 114.3 81.75625) (width 0.2) (layer "B.Cu") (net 13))
 (segment (start 114.3 81.75625) (end 114.3 66.675) (width 0.2) (layer "B.Cu") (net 13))
 (segment (start 120.015 95.09125) (end 120.015 78.022564) (width 0.2) (layer "B.Cu") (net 14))
 (segment (start 119.0625 60.0075) (end 119.0625 66.675) (width 0.2) (layer "B.Cu") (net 14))
 (segment (start 121.92 57.15) (end 119.0625 60.0075) (width 0.2) (layer "B.Cu") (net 14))
 (segment (start 118.614 76.621564) (end 118.614 67.1235) (width 0.2) (layer "B.Cu") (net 14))
 (segment (start 120.015 78.022564) (end 118.614 76.621564) (width 0.2) (layer "B.Cu") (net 14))
 (segment (start 119.0625 66.675) (end 118.614 67.1235) (width 0.2) (layer "B.Cu") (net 14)))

